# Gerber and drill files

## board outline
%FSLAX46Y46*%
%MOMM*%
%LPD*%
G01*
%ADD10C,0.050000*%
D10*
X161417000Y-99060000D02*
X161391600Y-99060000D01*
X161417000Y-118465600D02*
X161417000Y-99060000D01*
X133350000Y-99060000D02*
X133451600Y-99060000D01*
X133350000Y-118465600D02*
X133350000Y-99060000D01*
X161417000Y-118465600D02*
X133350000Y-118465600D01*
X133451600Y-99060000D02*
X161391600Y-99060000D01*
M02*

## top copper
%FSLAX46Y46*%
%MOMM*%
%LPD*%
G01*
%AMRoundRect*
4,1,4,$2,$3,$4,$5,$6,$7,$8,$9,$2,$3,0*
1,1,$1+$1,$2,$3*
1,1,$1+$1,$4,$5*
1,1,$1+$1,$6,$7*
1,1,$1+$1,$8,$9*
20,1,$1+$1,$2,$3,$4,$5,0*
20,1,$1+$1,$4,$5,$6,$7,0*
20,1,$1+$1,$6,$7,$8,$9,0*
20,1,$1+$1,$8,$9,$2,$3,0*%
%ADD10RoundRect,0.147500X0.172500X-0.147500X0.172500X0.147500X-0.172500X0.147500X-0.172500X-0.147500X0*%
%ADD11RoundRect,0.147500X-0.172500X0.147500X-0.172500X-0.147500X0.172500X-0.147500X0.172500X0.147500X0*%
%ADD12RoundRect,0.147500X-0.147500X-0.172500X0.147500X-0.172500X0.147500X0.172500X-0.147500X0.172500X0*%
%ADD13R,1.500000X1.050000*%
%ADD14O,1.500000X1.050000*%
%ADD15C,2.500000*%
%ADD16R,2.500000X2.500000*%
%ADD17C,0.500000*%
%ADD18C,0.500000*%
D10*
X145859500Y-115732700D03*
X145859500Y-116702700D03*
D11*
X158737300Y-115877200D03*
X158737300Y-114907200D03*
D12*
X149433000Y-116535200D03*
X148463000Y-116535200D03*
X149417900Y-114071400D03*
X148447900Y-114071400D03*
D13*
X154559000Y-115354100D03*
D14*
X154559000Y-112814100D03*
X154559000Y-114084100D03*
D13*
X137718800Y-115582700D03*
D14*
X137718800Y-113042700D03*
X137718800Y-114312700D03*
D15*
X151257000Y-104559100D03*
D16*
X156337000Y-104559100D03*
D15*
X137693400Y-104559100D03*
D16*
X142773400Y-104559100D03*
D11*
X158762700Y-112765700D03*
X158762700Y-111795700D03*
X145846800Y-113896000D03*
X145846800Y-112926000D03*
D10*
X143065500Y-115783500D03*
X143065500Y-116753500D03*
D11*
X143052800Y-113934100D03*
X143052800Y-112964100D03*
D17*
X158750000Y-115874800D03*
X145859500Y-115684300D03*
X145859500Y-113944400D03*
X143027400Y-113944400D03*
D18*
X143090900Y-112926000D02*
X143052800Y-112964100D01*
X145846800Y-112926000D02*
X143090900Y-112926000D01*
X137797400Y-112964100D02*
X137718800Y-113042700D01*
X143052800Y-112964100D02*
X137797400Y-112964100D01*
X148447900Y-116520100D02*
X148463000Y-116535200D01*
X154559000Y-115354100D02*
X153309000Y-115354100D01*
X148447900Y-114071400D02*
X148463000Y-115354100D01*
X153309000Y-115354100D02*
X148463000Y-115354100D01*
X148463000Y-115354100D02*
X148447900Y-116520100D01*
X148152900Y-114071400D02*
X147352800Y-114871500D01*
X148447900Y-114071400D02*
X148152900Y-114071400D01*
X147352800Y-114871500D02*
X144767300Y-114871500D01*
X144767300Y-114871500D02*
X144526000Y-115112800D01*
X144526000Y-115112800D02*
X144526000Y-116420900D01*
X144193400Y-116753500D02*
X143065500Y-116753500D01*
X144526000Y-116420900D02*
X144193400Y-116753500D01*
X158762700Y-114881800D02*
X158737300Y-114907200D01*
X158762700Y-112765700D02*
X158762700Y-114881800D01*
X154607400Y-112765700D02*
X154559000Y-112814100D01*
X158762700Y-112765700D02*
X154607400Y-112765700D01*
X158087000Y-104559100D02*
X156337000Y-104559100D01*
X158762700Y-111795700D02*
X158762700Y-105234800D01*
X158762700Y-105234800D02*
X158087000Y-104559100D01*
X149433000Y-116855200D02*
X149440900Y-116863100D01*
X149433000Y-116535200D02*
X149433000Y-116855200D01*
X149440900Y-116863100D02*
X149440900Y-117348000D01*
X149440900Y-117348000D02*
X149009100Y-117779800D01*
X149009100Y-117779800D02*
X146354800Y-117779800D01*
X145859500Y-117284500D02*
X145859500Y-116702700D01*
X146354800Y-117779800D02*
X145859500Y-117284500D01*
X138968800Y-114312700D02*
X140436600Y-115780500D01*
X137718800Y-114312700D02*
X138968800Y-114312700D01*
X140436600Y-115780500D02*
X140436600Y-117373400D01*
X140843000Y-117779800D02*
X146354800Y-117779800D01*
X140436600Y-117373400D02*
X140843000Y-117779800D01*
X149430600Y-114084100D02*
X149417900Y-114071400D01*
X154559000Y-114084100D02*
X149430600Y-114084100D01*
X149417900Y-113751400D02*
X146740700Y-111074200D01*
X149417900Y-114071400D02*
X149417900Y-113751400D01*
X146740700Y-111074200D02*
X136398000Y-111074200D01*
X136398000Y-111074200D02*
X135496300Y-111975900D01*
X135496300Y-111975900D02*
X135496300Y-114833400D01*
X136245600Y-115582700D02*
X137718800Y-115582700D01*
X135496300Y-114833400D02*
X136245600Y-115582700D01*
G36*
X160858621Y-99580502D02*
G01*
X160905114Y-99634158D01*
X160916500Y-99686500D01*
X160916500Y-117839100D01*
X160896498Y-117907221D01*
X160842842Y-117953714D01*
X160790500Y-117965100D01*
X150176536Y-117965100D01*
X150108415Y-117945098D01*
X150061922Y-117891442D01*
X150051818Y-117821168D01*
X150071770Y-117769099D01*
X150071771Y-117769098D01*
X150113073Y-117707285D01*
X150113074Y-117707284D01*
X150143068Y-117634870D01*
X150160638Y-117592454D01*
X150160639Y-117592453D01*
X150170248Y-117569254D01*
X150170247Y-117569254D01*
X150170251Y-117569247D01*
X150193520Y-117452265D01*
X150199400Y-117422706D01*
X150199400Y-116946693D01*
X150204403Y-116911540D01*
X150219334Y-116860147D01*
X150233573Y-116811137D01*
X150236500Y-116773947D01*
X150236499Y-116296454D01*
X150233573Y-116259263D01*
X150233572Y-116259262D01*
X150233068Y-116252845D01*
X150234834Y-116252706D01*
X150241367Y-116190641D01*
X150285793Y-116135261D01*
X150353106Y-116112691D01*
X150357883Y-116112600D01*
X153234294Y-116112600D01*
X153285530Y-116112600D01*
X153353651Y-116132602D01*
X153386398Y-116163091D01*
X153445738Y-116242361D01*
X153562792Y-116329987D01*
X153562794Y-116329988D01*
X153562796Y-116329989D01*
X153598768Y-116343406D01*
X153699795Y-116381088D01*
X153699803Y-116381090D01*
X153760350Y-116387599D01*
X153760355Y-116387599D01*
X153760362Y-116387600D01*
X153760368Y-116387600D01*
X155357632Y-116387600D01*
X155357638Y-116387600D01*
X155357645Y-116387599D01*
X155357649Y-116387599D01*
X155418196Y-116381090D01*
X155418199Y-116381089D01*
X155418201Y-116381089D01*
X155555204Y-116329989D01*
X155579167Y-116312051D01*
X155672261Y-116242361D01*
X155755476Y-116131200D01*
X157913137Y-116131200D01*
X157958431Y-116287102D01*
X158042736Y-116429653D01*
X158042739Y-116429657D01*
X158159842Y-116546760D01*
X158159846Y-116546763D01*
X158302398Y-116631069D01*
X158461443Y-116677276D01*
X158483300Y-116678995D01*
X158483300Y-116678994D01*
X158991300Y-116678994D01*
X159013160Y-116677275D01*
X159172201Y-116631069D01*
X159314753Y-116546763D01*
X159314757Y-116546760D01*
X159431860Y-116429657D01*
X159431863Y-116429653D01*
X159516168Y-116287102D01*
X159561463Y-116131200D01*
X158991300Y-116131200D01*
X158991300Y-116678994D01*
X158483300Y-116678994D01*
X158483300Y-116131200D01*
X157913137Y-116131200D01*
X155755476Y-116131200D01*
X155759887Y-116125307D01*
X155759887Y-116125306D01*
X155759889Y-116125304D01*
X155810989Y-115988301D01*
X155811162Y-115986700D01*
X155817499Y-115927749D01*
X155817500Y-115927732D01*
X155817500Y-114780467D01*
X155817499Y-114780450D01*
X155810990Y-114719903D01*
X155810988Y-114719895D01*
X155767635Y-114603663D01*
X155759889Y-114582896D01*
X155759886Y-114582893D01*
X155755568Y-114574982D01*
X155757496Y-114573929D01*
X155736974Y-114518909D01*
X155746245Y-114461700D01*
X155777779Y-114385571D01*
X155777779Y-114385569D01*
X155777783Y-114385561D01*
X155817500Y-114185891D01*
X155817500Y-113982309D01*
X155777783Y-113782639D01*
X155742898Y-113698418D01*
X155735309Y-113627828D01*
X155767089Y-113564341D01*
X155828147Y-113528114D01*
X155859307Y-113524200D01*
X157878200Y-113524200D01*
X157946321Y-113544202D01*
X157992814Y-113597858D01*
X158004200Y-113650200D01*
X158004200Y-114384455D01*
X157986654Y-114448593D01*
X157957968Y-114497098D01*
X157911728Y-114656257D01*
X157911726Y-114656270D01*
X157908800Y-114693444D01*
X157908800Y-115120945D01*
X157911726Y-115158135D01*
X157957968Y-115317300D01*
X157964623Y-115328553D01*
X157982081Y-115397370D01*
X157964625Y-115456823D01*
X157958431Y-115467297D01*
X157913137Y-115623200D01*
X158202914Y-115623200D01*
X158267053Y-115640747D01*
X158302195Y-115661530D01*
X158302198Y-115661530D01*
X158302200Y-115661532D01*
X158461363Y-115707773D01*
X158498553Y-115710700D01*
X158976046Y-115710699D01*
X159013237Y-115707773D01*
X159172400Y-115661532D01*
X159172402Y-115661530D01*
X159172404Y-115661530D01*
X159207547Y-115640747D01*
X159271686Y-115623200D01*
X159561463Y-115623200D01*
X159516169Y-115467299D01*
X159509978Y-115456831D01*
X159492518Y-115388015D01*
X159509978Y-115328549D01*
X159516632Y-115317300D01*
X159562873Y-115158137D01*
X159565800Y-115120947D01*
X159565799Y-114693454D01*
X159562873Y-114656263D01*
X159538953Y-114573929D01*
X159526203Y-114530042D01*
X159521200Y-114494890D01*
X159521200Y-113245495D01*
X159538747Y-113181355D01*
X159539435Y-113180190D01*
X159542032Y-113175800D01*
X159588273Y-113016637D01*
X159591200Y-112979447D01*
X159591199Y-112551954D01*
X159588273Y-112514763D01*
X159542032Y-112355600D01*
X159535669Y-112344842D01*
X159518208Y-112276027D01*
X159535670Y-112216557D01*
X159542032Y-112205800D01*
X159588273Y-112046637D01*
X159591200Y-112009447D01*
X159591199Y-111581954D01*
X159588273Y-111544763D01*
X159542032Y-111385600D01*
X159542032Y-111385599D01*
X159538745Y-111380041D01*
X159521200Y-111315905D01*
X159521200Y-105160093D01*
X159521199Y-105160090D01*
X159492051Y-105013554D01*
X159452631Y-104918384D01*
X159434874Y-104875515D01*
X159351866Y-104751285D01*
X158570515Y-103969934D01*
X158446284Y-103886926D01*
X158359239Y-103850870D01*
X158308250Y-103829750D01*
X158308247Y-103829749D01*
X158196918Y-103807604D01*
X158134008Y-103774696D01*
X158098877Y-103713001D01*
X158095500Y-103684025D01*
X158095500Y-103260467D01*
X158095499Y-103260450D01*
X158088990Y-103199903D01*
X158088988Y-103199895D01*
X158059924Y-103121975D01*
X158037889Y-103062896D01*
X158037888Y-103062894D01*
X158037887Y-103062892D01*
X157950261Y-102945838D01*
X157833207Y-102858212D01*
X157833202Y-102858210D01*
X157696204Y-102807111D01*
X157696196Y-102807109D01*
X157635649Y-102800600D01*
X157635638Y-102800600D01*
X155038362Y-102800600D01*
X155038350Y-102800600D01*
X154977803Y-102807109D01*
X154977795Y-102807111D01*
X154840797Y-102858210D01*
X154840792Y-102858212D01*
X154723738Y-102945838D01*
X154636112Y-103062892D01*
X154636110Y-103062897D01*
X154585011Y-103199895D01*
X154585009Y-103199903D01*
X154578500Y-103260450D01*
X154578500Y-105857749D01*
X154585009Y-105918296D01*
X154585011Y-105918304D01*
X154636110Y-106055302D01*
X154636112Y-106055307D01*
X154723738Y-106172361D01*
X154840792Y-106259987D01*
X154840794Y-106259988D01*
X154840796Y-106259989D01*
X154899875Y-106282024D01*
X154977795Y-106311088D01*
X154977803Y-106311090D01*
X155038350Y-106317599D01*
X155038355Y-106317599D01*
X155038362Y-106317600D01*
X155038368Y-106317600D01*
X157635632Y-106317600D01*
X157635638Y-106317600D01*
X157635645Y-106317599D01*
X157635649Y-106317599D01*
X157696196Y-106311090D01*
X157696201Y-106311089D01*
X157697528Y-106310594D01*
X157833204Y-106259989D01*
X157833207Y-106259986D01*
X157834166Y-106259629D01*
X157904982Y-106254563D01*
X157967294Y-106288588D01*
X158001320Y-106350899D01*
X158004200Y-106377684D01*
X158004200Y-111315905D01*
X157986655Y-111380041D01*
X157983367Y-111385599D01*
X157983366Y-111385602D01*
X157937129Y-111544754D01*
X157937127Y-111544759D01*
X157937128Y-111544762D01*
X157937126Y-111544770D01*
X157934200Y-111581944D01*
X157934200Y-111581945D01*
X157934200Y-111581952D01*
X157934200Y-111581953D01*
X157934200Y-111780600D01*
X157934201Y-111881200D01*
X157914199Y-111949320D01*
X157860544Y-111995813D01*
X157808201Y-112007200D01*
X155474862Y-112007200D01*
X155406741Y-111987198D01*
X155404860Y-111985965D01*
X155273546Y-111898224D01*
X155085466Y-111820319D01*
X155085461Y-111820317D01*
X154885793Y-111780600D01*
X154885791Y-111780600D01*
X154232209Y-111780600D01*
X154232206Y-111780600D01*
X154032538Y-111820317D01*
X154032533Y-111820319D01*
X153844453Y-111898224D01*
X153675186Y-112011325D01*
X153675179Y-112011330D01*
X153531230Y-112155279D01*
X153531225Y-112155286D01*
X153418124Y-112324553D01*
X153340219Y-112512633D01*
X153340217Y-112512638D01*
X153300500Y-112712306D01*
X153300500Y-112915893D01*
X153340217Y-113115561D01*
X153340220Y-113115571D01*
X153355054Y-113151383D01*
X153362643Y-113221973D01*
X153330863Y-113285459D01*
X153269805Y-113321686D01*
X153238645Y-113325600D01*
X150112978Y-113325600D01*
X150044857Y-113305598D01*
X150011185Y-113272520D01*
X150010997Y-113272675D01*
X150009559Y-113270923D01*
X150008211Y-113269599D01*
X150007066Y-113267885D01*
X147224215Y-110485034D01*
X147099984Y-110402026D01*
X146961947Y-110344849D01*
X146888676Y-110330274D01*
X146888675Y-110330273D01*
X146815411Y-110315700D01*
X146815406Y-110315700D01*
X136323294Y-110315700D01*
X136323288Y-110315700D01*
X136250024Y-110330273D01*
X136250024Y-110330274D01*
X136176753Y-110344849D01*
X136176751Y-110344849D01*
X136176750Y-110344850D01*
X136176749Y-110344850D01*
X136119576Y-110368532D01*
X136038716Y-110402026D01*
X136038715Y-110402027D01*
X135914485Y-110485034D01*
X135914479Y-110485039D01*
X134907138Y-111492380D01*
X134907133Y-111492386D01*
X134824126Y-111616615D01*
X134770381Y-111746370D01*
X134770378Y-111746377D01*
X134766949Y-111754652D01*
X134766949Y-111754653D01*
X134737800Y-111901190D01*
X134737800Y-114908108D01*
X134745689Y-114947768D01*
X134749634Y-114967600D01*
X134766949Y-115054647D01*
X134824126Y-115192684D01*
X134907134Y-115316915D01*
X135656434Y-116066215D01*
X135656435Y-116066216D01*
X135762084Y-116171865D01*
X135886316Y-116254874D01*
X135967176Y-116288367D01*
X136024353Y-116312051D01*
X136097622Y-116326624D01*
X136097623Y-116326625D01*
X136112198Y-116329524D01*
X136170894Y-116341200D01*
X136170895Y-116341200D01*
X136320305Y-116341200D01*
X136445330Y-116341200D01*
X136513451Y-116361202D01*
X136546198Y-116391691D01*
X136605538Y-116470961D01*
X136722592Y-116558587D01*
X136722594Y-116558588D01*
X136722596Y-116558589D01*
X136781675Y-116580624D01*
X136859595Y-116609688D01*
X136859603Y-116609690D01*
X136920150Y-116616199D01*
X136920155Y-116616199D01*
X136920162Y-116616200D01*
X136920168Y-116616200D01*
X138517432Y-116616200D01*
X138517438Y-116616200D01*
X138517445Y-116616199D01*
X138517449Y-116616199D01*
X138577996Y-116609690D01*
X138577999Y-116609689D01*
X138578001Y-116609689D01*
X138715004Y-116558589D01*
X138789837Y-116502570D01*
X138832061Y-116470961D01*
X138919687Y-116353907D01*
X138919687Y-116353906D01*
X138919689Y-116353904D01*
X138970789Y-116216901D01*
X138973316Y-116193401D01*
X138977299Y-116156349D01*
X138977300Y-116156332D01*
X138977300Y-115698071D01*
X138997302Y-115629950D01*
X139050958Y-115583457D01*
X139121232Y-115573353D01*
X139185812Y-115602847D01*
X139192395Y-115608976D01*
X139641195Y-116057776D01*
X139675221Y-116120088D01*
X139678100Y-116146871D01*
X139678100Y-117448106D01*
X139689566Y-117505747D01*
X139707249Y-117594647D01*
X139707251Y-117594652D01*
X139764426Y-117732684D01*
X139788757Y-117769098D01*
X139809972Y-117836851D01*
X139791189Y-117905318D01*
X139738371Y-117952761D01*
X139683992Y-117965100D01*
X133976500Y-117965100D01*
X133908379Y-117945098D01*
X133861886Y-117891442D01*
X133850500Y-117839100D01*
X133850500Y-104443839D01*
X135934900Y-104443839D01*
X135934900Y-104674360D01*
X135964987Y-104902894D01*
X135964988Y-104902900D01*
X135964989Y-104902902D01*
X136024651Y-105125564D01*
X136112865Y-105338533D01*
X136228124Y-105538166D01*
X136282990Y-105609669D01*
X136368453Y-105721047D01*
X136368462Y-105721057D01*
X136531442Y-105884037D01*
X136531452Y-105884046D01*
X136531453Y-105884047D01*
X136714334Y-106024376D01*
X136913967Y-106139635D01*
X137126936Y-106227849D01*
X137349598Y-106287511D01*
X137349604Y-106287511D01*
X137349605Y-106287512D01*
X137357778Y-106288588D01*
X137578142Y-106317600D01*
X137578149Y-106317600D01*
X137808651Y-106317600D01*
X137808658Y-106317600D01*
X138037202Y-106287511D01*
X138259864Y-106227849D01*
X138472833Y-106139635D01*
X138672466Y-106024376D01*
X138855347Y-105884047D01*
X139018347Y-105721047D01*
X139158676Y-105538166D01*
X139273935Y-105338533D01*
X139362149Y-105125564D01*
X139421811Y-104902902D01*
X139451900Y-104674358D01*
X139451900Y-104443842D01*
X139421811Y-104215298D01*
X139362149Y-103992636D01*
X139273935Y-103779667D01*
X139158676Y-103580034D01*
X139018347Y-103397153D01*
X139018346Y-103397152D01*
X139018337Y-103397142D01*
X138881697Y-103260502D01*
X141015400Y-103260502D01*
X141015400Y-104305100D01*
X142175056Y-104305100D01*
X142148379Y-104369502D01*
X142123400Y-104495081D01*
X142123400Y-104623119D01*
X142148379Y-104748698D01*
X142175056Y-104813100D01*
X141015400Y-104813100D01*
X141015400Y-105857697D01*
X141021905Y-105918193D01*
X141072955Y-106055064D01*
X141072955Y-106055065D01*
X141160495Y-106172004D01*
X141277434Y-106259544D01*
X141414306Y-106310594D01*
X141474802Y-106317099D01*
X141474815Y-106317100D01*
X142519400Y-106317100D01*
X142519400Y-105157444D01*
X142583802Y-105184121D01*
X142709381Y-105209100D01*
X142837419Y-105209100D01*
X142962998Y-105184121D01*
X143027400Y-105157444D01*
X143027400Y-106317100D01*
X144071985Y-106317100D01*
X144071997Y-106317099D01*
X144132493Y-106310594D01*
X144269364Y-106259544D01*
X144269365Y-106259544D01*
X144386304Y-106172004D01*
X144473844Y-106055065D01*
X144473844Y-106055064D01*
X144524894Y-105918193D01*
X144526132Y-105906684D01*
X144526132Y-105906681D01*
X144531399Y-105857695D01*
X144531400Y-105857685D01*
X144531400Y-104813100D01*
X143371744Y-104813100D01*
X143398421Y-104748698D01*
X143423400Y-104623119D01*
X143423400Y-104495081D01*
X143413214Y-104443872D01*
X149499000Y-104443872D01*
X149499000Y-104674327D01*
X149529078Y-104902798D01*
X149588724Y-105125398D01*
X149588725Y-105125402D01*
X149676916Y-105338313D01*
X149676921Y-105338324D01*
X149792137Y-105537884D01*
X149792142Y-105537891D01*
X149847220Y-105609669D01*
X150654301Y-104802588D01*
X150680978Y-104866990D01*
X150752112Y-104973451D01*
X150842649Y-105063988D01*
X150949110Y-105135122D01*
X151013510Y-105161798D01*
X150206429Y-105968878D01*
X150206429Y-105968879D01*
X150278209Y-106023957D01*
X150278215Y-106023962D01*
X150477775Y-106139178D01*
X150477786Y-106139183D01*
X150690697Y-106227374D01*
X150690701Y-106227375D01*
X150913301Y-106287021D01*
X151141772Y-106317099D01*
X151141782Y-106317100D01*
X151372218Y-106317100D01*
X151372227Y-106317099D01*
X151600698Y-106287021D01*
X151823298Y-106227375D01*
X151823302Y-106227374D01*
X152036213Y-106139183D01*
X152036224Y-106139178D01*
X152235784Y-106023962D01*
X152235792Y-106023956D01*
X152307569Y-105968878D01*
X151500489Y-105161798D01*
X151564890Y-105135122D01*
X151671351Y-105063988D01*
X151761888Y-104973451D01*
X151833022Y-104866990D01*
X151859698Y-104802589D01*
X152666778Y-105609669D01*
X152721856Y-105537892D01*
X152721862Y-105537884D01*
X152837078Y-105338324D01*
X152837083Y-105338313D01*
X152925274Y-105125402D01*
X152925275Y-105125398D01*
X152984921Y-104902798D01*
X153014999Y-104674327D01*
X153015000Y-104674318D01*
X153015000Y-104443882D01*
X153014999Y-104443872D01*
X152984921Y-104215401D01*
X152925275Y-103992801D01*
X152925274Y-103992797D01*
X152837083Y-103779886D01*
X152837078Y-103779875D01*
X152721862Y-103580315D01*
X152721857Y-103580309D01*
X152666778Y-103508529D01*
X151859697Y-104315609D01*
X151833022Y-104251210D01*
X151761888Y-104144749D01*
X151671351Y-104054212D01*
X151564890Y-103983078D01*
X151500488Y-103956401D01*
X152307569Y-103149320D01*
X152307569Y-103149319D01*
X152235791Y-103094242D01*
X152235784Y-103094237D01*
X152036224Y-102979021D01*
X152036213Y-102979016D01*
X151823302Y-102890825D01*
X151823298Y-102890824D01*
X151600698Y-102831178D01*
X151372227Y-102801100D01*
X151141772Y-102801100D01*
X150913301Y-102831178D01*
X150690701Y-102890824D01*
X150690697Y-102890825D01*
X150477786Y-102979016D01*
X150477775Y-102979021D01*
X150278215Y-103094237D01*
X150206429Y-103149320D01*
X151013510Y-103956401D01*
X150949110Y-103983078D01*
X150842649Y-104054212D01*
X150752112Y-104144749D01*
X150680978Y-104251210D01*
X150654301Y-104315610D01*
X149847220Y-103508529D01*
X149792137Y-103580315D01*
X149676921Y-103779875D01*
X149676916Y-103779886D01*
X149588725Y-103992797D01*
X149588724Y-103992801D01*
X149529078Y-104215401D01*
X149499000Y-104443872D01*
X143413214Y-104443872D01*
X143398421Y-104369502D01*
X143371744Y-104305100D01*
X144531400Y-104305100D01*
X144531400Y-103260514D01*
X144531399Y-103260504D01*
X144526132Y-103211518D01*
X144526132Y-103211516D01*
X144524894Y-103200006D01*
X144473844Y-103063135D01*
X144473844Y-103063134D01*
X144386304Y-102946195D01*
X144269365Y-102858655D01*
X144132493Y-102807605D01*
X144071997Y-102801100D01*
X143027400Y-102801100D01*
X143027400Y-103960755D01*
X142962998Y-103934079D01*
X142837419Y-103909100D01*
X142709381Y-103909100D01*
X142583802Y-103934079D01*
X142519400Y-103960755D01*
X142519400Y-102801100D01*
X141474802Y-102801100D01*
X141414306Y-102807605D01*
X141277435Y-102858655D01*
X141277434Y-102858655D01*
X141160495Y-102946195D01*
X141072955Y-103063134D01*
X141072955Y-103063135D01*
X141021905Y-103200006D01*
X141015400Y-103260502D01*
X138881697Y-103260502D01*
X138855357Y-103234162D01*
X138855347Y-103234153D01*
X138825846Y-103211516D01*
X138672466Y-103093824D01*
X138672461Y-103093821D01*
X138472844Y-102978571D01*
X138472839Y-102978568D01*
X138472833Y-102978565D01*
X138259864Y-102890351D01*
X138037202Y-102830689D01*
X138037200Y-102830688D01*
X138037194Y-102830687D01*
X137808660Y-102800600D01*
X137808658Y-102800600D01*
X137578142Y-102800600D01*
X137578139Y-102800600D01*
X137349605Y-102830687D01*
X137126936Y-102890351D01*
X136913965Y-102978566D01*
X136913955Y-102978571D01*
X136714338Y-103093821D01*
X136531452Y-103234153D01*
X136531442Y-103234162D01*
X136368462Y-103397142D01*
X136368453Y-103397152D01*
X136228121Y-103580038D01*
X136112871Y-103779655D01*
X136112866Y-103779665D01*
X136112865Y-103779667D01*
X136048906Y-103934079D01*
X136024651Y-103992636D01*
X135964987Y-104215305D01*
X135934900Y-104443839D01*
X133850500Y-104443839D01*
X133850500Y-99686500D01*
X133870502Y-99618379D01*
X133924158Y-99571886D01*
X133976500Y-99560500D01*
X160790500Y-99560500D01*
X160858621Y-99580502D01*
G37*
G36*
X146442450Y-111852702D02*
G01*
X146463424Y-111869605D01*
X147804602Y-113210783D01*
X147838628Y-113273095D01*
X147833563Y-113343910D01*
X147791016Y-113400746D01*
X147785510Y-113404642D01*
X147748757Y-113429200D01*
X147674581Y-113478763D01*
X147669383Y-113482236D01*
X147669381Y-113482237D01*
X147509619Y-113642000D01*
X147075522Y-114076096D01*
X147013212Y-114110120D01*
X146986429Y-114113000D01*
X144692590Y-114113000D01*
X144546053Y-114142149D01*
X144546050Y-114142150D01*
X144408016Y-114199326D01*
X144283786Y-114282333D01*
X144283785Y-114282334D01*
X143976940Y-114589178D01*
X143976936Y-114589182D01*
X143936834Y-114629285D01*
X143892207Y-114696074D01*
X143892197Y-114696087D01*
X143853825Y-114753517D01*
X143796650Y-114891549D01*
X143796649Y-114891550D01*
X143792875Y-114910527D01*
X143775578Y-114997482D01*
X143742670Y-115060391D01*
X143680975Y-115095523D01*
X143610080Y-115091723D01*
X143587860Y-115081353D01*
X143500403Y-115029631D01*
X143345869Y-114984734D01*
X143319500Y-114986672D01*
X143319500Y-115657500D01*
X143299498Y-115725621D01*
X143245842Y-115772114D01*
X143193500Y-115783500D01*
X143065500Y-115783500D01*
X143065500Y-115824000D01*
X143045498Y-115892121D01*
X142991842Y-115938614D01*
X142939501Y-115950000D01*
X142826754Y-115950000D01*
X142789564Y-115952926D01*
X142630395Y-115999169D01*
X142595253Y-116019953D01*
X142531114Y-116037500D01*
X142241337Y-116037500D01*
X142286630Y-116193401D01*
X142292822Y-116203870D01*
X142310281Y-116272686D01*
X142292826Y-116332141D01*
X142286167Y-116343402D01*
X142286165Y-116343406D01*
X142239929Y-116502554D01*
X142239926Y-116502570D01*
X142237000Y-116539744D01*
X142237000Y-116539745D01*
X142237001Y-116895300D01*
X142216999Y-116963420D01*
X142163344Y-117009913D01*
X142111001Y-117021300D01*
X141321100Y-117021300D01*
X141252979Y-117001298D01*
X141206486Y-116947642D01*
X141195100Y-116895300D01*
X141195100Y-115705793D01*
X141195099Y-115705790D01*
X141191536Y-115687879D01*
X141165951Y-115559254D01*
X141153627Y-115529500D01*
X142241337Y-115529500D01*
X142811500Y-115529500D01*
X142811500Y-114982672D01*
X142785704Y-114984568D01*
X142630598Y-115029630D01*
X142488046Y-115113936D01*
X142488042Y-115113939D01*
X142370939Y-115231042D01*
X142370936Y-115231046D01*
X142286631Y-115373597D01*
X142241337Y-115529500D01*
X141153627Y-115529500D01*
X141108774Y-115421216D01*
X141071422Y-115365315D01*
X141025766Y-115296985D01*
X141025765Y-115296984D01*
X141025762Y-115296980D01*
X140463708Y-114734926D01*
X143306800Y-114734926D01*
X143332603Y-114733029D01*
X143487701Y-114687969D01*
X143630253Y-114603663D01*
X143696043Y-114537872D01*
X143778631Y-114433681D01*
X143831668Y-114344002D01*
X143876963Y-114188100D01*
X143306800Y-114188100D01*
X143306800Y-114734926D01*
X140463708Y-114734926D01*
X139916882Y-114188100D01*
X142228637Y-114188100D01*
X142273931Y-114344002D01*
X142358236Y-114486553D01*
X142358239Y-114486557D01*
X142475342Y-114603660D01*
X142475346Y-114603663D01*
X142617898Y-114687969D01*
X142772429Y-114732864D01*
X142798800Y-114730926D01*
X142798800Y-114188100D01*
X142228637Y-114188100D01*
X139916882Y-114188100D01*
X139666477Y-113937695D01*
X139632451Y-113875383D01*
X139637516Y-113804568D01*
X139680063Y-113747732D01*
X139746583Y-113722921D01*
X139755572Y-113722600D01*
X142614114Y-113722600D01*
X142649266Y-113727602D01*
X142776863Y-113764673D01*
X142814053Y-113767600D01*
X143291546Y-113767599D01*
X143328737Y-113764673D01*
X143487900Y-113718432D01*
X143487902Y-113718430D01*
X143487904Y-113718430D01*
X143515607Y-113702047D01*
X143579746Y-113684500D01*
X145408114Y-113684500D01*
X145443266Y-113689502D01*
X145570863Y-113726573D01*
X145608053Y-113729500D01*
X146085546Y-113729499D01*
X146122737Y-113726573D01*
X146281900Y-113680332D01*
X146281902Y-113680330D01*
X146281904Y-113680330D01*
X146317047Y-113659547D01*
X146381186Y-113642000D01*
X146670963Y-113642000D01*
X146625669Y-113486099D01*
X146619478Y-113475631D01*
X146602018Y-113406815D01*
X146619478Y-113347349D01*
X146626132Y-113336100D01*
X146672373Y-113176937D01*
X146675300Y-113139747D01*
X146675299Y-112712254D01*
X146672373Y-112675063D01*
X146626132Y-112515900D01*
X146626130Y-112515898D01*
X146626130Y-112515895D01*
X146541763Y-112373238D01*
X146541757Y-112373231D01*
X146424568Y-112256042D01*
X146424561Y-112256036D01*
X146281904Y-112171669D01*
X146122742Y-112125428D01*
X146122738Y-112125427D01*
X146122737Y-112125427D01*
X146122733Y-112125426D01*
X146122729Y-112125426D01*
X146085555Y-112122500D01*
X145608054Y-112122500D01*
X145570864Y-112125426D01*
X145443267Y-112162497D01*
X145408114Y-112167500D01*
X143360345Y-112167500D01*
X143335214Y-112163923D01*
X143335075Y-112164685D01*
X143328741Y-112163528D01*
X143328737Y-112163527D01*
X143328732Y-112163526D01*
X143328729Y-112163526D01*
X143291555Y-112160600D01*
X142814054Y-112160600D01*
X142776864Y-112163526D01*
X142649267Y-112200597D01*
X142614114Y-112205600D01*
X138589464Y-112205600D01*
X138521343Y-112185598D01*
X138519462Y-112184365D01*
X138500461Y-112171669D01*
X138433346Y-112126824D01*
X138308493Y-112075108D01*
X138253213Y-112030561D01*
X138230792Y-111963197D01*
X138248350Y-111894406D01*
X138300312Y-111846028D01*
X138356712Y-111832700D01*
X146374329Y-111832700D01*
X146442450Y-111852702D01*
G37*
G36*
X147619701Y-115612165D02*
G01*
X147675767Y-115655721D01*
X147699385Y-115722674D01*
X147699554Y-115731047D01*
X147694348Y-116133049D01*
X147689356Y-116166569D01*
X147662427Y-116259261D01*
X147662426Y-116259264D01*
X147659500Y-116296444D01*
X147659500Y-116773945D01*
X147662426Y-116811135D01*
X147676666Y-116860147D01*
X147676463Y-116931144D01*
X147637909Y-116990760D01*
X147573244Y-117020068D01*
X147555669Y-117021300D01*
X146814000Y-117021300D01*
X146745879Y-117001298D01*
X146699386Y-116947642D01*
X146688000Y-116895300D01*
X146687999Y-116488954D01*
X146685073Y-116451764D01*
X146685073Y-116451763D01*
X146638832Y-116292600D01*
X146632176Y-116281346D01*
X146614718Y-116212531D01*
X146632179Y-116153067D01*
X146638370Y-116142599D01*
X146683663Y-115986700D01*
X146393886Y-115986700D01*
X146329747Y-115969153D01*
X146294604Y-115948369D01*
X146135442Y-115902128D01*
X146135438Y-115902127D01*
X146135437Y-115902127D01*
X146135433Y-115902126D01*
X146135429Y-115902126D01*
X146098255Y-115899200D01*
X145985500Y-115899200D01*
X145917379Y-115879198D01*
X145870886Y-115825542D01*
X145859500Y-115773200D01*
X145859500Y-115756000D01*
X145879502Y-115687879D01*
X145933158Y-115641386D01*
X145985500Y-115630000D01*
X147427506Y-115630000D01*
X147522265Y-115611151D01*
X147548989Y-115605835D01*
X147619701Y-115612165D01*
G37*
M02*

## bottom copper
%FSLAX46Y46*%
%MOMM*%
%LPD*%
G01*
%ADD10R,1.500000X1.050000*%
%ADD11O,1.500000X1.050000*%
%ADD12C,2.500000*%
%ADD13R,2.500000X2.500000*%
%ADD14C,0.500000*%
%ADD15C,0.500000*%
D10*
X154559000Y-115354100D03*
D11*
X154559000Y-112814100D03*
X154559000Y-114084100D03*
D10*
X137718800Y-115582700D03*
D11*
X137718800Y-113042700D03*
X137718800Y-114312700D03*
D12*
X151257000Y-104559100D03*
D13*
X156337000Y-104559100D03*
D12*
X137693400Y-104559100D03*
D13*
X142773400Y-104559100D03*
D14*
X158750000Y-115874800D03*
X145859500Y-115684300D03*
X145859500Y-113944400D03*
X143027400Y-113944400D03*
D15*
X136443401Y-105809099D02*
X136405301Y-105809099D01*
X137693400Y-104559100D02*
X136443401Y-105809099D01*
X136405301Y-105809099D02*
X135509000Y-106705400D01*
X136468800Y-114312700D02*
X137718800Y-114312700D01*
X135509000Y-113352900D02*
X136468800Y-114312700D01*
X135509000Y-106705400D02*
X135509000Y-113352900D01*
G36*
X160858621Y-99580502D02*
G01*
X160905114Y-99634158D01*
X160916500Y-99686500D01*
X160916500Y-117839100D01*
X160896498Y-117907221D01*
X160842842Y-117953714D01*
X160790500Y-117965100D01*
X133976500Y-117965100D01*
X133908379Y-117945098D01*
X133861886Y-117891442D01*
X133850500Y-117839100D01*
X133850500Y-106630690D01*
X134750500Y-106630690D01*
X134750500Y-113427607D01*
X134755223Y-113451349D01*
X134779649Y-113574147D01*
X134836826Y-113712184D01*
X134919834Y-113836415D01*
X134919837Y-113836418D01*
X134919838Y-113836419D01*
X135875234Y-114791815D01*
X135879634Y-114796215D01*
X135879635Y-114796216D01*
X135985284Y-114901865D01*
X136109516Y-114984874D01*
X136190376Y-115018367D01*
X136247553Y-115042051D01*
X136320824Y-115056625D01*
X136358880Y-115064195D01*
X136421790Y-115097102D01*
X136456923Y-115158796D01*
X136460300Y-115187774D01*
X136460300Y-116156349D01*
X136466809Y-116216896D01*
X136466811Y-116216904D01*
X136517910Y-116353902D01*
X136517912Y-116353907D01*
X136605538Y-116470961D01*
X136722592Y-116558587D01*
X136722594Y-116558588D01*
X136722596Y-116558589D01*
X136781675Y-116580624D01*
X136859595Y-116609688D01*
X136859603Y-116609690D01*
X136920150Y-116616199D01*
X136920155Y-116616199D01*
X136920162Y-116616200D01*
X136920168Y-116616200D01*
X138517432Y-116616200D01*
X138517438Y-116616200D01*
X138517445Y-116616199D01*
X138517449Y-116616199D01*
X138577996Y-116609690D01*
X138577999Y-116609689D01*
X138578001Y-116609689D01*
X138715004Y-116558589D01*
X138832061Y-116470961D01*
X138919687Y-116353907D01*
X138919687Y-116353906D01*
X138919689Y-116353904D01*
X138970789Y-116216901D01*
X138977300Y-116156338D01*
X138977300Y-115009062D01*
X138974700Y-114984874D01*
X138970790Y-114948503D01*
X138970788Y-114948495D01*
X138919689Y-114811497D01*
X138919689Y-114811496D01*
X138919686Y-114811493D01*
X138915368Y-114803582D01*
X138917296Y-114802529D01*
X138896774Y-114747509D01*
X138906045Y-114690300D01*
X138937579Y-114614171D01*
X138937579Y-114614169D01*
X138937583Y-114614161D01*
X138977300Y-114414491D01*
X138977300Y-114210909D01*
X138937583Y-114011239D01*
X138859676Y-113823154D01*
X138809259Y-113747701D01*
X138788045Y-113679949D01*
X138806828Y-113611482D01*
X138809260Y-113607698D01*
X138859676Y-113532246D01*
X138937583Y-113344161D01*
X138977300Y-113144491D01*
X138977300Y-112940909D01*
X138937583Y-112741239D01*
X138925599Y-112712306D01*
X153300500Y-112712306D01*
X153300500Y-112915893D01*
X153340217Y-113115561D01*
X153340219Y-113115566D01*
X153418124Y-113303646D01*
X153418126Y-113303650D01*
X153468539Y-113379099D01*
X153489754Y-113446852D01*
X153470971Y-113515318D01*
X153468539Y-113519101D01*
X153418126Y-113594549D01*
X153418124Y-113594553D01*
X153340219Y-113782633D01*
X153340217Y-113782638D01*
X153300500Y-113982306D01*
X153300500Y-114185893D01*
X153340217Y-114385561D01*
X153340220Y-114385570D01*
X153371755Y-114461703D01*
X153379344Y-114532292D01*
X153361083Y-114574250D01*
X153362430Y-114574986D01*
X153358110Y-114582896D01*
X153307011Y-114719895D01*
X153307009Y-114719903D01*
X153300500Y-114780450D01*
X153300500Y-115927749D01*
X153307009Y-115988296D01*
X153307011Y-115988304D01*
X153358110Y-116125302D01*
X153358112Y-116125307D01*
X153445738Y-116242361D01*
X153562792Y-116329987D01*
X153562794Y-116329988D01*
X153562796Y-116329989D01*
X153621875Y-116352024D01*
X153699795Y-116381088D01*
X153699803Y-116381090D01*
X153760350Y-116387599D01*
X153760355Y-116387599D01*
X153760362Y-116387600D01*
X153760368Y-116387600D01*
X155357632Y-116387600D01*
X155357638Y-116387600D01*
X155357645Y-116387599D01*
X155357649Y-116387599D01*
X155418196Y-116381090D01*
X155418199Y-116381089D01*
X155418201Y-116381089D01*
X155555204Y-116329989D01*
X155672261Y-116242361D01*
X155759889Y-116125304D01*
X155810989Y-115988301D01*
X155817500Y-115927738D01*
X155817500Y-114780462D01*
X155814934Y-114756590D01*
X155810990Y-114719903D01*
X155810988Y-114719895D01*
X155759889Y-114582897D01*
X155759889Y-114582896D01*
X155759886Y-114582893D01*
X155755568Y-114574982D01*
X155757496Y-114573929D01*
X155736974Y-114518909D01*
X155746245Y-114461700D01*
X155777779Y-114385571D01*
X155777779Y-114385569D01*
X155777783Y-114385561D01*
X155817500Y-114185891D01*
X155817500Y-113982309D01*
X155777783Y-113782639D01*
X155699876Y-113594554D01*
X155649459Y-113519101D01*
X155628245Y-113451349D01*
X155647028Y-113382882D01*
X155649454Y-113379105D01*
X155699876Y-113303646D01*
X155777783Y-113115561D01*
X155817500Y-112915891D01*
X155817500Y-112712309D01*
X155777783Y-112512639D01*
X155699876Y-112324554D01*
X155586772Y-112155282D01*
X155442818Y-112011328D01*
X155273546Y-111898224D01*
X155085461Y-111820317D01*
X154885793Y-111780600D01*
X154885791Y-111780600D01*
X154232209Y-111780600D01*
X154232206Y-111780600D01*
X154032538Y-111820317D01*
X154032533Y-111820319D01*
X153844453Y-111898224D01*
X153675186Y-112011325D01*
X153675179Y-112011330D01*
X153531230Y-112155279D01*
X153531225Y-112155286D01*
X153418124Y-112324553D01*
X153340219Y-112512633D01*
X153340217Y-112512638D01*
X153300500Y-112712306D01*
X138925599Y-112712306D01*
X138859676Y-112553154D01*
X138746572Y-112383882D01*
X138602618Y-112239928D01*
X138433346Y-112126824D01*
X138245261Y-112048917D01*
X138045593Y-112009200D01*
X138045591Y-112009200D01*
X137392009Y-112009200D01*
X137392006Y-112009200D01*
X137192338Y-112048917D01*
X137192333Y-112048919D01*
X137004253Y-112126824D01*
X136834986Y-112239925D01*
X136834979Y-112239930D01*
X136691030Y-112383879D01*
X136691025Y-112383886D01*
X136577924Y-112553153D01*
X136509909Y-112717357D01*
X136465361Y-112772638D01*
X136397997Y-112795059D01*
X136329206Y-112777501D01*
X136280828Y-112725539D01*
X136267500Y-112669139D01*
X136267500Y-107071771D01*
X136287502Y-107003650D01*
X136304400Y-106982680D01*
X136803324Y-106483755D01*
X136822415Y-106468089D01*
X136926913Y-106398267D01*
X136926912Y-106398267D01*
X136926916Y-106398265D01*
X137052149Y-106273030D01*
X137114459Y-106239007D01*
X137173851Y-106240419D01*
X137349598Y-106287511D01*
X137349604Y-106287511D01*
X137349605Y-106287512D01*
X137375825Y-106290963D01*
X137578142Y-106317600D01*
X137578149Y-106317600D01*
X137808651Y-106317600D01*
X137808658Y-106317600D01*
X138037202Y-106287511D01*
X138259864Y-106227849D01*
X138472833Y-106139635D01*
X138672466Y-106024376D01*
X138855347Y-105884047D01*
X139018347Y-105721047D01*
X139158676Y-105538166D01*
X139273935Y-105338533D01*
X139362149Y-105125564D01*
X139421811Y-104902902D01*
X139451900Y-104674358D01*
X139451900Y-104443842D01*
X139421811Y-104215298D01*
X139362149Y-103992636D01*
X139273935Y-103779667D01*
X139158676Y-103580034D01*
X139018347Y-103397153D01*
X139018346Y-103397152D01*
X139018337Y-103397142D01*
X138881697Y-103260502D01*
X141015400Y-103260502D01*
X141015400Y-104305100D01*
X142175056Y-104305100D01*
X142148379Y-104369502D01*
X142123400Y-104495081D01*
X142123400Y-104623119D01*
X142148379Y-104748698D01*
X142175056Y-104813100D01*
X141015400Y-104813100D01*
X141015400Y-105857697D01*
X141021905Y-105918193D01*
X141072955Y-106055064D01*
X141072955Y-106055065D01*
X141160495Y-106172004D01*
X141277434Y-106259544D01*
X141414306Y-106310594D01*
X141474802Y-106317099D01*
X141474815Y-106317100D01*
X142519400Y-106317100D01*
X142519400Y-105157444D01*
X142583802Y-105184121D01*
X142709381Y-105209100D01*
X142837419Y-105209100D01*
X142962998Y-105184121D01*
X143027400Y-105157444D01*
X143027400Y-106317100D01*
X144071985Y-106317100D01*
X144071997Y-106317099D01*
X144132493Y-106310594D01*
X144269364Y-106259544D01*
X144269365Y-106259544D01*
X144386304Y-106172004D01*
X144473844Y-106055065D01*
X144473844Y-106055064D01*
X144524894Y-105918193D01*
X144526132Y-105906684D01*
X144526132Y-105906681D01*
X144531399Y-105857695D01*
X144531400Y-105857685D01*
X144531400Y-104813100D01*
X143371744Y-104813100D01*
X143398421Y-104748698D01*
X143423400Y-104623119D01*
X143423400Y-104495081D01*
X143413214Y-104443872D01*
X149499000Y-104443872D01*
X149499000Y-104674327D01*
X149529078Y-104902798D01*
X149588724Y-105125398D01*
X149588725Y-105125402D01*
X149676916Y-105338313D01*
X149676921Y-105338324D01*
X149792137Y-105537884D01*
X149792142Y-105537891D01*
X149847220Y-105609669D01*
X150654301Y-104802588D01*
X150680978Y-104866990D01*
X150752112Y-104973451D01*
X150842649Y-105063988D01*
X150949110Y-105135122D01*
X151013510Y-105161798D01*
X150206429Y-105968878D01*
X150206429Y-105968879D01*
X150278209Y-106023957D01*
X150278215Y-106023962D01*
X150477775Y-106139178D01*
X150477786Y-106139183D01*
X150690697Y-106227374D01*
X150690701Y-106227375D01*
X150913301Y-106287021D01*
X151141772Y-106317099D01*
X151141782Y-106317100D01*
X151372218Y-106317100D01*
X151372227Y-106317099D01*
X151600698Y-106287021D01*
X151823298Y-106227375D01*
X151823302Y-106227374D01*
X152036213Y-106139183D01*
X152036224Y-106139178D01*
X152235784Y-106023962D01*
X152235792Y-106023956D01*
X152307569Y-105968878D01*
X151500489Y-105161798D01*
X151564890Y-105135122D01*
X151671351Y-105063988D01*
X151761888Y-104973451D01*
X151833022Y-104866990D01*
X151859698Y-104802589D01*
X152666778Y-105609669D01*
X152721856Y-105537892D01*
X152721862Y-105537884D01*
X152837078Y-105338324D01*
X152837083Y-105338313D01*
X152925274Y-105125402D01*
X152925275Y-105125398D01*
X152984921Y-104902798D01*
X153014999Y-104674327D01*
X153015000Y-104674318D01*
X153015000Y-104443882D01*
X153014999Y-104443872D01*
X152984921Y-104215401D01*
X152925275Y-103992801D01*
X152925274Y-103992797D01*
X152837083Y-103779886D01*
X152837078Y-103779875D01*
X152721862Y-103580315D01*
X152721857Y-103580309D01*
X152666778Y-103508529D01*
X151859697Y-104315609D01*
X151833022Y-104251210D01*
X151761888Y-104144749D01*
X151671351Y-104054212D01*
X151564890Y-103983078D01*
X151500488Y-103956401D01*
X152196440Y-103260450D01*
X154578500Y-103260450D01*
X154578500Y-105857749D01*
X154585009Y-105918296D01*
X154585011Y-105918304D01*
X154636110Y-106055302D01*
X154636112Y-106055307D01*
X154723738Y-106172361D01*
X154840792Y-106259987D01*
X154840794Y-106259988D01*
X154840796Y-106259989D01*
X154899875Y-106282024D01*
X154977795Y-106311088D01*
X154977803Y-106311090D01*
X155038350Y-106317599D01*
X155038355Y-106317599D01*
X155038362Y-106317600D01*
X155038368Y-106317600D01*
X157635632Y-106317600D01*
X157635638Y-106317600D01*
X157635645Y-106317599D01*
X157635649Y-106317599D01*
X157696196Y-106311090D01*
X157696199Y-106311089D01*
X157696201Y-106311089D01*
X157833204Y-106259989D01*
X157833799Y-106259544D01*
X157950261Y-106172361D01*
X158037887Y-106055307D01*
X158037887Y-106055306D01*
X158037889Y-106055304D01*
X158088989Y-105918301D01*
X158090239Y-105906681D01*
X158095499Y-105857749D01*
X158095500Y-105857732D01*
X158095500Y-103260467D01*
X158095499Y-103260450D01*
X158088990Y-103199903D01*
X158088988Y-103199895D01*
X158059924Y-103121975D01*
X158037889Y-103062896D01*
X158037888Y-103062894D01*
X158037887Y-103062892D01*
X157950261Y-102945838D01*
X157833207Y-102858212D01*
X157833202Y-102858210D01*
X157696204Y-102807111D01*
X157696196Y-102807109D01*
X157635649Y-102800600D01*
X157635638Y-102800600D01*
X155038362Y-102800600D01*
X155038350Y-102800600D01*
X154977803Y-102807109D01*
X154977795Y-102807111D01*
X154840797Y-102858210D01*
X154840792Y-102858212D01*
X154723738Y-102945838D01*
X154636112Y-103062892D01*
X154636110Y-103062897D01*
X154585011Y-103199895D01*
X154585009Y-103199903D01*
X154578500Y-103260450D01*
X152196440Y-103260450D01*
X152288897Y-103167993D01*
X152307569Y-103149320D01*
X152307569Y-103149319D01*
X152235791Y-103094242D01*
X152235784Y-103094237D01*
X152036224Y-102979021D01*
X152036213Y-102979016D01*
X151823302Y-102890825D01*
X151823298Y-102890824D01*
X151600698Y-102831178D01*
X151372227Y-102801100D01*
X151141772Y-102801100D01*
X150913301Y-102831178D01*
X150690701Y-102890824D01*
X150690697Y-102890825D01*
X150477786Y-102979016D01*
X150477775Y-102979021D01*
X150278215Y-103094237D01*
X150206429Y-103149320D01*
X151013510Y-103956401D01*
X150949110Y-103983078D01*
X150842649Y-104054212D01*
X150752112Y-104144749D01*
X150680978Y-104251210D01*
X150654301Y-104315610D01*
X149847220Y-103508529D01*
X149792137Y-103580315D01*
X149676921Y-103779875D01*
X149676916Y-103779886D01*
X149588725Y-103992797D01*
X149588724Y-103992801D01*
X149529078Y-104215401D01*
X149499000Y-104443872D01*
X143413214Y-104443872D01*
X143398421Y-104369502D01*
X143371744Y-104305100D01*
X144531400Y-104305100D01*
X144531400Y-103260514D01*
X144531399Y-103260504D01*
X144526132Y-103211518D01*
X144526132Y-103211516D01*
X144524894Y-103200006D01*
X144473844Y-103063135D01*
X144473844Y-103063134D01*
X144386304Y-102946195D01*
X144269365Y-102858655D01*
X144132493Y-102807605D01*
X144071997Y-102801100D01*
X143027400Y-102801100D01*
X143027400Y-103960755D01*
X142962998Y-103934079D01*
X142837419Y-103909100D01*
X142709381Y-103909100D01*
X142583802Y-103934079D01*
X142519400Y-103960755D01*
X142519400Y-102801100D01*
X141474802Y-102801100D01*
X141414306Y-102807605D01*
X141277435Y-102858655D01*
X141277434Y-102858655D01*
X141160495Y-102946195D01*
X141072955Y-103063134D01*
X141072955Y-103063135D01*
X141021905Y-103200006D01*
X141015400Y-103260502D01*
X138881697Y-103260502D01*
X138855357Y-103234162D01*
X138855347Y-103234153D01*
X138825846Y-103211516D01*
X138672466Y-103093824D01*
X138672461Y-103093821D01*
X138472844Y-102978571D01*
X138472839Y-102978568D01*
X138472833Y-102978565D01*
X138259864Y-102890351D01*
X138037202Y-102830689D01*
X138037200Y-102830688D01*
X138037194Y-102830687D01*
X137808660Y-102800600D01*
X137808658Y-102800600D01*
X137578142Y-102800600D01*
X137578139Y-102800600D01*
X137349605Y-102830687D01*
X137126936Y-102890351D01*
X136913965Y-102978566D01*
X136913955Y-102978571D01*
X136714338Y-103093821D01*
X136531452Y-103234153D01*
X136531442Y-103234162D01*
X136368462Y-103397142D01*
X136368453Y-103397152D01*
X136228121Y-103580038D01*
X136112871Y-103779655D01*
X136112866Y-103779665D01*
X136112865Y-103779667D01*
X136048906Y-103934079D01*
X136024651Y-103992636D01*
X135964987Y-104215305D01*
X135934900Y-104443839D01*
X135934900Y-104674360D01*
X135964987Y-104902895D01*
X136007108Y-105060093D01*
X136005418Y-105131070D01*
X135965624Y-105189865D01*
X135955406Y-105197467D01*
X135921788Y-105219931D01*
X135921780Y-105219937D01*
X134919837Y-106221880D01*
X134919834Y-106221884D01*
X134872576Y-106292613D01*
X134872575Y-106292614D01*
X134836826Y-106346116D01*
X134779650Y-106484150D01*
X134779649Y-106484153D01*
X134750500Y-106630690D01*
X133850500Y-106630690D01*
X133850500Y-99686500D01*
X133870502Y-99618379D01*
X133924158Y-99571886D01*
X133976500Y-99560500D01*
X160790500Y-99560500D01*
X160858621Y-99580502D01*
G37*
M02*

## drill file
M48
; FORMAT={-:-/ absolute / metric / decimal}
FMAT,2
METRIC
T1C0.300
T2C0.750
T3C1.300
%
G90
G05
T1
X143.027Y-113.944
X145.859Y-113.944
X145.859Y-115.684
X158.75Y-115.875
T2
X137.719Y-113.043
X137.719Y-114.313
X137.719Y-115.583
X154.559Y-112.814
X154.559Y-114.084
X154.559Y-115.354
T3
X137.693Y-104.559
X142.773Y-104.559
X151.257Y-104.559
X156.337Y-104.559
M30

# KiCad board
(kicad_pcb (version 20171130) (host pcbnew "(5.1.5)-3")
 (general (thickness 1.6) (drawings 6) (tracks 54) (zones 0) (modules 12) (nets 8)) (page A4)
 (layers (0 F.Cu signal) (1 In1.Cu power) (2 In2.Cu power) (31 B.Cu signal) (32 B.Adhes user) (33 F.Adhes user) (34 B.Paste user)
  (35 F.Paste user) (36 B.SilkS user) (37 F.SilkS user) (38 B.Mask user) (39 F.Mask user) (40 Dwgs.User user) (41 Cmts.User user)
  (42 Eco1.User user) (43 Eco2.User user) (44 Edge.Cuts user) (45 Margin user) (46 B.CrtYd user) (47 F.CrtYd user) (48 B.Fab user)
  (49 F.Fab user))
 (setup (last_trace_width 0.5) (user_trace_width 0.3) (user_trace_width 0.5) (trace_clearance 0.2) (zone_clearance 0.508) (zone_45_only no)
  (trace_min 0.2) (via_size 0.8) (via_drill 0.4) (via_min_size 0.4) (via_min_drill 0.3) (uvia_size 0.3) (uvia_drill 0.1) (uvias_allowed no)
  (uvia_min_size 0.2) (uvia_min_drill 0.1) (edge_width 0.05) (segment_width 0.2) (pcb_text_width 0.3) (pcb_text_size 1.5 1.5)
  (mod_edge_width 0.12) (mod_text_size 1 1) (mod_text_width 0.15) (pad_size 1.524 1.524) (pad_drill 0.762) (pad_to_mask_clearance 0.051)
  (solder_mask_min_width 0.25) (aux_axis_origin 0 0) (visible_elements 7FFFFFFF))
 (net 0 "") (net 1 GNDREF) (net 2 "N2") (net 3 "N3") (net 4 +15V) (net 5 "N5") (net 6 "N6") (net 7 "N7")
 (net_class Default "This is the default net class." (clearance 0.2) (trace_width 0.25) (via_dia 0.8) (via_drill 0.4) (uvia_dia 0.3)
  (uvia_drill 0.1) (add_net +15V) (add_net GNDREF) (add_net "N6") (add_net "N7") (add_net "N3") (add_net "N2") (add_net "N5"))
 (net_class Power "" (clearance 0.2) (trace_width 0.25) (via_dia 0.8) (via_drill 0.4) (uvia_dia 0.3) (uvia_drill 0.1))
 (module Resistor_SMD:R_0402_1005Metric (layer F.Cu) (at 145.8595 116.2177 90)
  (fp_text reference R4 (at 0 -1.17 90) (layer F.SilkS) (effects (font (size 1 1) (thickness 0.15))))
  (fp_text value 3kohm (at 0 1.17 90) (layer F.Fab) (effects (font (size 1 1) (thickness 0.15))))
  (pad 2 smd roundrect (at 0.485 0 90) (size 0.59 0.64) (layers F.Cu F.Paste F.Mask) (roundrect_rratio 0.25) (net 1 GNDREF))
  (pad 1 smd roundrect (at -0.485 0 90) (size 0.59 0.64) (layers F.Cu F.Paste F.Mask) (roundrect_rratio 0.25) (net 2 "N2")))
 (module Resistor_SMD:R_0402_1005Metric (layer F.Cu) (at 158.7373 115.3922 270)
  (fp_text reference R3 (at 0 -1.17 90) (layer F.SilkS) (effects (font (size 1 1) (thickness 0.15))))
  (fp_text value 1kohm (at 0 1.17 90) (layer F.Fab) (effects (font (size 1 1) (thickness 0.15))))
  (pad 2 smd roundrect (at 0.485 0 270) (size 0.59 0.64) (layers F.Cu F.Paste F.Mask) (roundrect_rratio 0.25) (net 1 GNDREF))
  (pad 1 smd roundrect (at -0.485 0 270) (size 0.59 0.64) (layers F.Cu F.Paste F.Mask) (roundrect_rratio 0.25) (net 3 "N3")))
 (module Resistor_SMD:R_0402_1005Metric (layer F.Cu) (at 148.948 116.5352)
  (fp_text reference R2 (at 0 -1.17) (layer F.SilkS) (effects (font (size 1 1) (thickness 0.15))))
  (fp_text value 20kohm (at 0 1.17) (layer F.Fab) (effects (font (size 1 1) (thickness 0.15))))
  (pad 2 smd roundrect (at 0.485 0) (size 0.59 0.64) (layers F.Cu F.Paste F.Mask) (roundrect_rratio 0.25) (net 2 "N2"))
  (pad 1 smd roundrect (at -0.485 0) (size 0.59 0.64) (layers F.Cu F.Paste F.Mask) (roundrect_rratio 0.25) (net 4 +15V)))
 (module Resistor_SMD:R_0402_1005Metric (layer F.Cu) (at 148.9329 114.0714)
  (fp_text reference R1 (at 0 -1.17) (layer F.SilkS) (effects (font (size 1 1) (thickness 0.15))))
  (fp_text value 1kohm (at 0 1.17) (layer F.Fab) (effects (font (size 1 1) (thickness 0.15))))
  (pad 2 smd roundrect (at 0.485 0) (size 0.59 0.64) (layers F.Cu F.Paste F.Mask) (roundrect_rratio 0.25) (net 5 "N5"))
  (pad 1 smd roundrect (at -0.485 0) (size 0.59 0.64) (layers F.Cu F.Paste F.Mask) (roundrect_rratio 0.25) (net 4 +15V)))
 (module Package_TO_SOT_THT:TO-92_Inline (layer F.Cu) (at 154.559 115.3541 90)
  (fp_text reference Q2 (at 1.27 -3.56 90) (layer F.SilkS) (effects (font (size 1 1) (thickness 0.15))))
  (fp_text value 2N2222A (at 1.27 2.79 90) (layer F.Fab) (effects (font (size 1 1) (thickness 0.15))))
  (pad 1 thru_hole rect (at 0 0 90) (size 1.05 1.5) (drill 0.75) (layers *.Cu *.Mask) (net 4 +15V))
  (pad 3 thru_hole oval (at 2.54 0 90) (size 1.05 1.5) (drill 0.75) (layers *.Cu *.Mask) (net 3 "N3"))
  (pad 2 thru_hole oval (at 1.27 0 90) (size 1.05 1.5) (drill 0.75) (layers *.Cu *.Mask) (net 5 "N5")))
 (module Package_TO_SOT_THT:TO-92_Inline (layer F.Cu) (at 137.7188 115.5827 90)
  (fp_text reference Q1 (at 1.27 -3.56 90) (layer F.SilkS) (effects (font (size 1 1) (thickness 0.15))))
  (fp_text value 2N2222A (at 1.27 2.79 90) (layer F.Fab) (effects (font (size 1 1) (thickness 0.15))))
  (pad 1 thru_hole rect (at 0 0 90) (size 1.05 1.5) (drill 0.75) (layers *.Cu *.Mask) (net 5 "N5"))
  (pad 3 thru_hole oval (at 2.54 0 90) (size 1.05 1.5) (drill 0.75) (layers *.Cu *.Mask) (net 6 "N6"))
  (pad 2 thru_hole oval (at 1.27 0 90) (size 1.05 1.5) (drill 0.75) (layers *.Cu *.Mask) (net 2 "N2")))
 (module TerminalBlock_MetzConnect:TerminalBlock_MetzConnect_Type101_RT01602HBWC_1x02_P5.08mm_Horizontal (layer F.Cu)
  (at 156.337 104.5591 180)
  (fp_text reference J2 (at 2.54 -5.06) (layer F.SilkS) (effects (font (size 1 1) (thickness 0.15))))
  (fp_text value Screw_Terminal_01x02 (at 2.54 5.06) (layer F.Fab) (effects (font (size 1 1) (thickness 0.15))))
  (pad 2 thru_hole circle (at 5.08 0 180) (size 2.5 2.5) (drill 1.3) (layers *.Cu *.Mask) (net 1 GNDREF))
  (pad 1 thru_hole rect (at 0 0 180) (size 2.5 2.5) (drill 1.3) (layers *.Cu *.Mask) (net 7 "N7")))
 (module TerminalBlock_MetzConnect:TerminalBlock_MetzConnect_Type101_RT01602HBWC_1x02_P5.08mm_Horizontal (layer F.Cu)
  (at 142.7734 104.5591 180)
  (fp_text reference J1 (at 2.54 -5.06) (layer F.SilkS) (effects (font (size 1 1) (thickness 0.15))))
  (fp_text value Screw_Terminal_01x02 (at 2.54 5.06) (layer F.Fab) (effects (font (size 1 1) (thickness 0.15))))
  (pad 2 thru_hole circle (at 5.08 0 180) (size 2.5 2.5) (drill 1.3) (layers *.Cu *.Mask) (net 2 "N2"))
  (pad 1 thru_hole rect (at 0 0 180) (size 2.5 2.5) (drill 1.3) (layers *.Cu *.Mask) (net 1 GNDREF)))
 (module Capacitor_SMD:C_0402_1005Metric (layer F.Cu) (at 158.7627 112.2807 270)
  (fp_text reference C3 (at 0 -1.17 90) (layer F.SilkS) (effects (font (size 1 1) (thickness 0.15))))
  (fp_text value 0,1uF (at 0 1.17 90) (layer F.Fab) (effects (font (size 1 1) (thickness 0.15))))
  (pad 2 smd roundrect (at 0.485 0 270) (size 0.59 0.64) (layers F.Cu F.Paste F.Mask) (roundrect_rratio 0.25) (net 3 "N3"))
  (pad 1 smd roundrect (at -0.485 0 270) (size 0.59 0.64) (layers F.Cu F.Paste F.Mask) (roundrect_rratio 0.25) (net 7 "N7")))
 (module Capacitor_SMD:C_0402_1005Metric (layer F.Cu) (at 145.8468 113.411 270)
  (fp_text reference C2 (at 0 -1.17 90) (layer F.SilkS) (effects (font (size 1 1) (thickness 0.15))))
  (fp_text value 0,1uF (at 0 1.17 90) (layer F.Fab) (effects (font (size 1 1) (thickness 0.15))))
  (pad 2 smd roundrect (at 0.485 0 270) (size 0.59 0.64) (layers F.Cu F.Paste F.Mask) (roundrect_rratio 0.25) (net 1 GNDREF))
  (pad 1 smd roundrect (at -0.485 0 270) (size 0.59 0.64) (layers F.Cu F.Paste F.Mask) (roundrect_rratio 0.25) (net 6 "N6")))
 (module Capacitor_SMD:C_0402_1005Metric (layer F.Cu) (at 143.0655 116.2685 90)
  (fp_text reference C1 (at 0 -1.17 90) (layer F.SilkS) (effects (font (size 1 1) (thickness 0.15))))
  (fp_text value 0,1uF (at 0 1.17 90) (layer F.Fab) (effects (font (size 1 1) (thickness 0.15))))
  (pad 2 smd roundrect (at 0.485 0 90) (size 0.59 0.64) (layers F.Cu F.Paste F.Mask) (roundrect_rratio 0.25) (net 1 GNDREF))
  (pad 1 smd roundrect (at -0.485 0 90) (size 0.59 0.64) (layers F.Cu F.Paste F.Mask) (roundrect_rratio 0.25) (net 4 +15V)))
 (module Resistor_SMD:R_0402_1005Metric (layer F.Cu) (at 143.0528 113.4491 270)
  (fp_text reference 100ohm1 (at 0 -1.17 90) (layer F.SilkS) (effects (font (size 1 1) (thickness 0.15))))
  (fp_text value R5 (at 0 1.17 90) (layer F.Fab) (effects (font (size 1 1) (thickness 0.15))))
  (pad 2 smd roundrect (at 0.485 0 270) (size 0.59 0.64) (layers F.Cu F.Paste F.Mask) (roundrect_rratio 0.25) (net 1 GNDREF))
  (pad 1 smd roundrect (at -0.485 0 270) (size 0.59 0.64) (layers F.Cu F.Paste F.Mask) (roundrect_rratio 0.25) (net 6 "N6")))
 (gr_line (start 161.417 99.06) (end 161.3916 99.06) (layer Edge.Cuts) (width 0.05))
 (gr_line (start 161.417 118.4656) (end 161.417 99.06) (layer Edge.Cuts) (width 0.05))
 (gr_line (start 133.35 99.06) (end 133.4516 99.06) (layer Edge.Cuts) (width 0.05))
 (gr_line (start 133.35 118.4656) (end 133.35 99.06) (layer Edge.Cuts) (width 0.05))
 (gr_line (start 161.417 118.4656) (end 133.35 118.4656) (layer Edge.Cuts) (width 0.05))
 (gr_line (start 133.4516 99.06) (end 161.3916 99.06) (layer Edge.Cuts) (width 0.05))
 (via (at 158.75 115.8748) (size 0.5) (drill 0.3) (layers F.Cu B.Cu) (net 1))
 (via (at 145.8595 115.6843) (size 0.5) (drill 0.3) (layers F.Cu B.Cu) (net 1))
 (via (at 145.8595 113.9444) (size 0.5) (drill 0.3) (layers F.Cu B.Cu) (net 1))
 (via (at 143.0274 113.9444) (size 0.5) (drill 0.3) (layers F.Cu B.Cu) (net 1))
 (segment (start 143.0909 112.926) (end 143.0528 112.9641) (width 0.5) (layer F.Cu) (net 6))
 (segment (start 145.8468 112.926) (end 143.0909 112.926) (width 0.5) (layer F.Cu) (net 6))
 (segment (start 137.7974 112.9641) (end 137.7188 113.0427) (width 0.5) (layer F.Cu) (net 6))
 (segment (start 143.0528 112.9641) (end 137.7974 112.9641) (width 0.5) (layer F.Cu) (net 6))
 (segment (start 148.4479 116.5201) (end 148.463 116.5352) (width 0.5) (layer F.Cu) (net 4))
 (segment (start 154.559 115.3541) (end 153.309 115.3541) (width 0.5) (layer F.Cu) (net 4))
 (segment (start 148.4479 114.0714) (end 148.463 115.3541) (width 0.5) (layer F.Cu) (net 4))
 (segment (start 153.309 115.3541) (end 148.463 115.3541) (width 0.5) (layer F.Cu) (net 4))
 (segment (start 148.463 115.3541) (end 148.4479 116.5201) (width 0.5) (layer F.Cu) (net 4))
 (segment (start 148.1529 114.0714) (end 147.3528 114.8715) (width 0.5) (layer F.Cu) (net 4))
 (segment (start 148.4479 114.0714) (end 148.1529 114.0714) (width 0.5) (layer F.Cu) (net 4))
 (segment (start 147.3528 114.8715) (end 144.7673 114.8715) (width 0.5) (layer F.Cu) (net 4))
 (segment (start 144.7673 114.8715) (end 144.526 115.1128) (width 0.5) (layer F.Cu) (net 4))
 (segment (start 144.526 115.1128) (end 144.526 116.4209) (width 0.5) (layer F.Cu) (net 4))
 (segment (start 144.1934 116.7535) (end 143.0655 116.7535) (width 0.5) (layer F.Cu) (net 4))
 (segment (start 144.526 116.4209) (end 144.1934 116.7535) (width 0.5) (layer F.Cu) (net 4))
 (segment (start 158.7627 114.8818) (end 158.7373 114.9072) (width 0.5) (layer F.Cu) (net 3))
 (segment (start 158.7627 112.7657) (end 158.7627 114.8818) (width 0.5) (layer F.Cu) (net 3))
 (segment (start 154.6074 112.7657) (end 154.559 112.8141) (width 0.5) (layer F.Cu) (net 3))
 (segment (start 158.7627 112.7657) (end 154.6074 112.7657) (width 0.5) (layer F.Cu) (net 3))
 (segment (start 158.087 104.5591) (end 156.337 104.5591) (width 0.5) (layer F.Cu) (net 7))
 (segment (start 158.7627 111.7957) (end 158.7627 105.2348) (width 0.5) (layer F.Cu) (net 7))
 (segment (start 158.7627 105.2348) (end 158.087 104.5591) (width 0.5) (layer F.Cu) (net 7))
 (segment (start 136.443401 105.809099) (end 136.405301 105.809099) (width 0.5) (layer B.Cu) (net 2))
 (segment (start 137.6934 104.5591) (end 136.443401 105.809099) (width 0.5) (layer B.Cu) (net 2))
 (segment (start 136.405301 105.809099) (end 135.509 106.7054) (width 0.5) (layer B.Cu) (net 2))
 (segment (start 136.4688 114.3127) (end 137.7188 114.3127) (width 0.5) (layer B.Cu) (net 2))
 (segment (start 135.509 113.3529) (end 136.4688 114.3127) (width 0.5) (layer B.Cu) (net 2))
 (segment (start 135.509 106.7054) (end 135.509 113.3529) (width 0.5) (layer B.Cu) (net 2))
 (segment (start 149.433 116.8552) (end 149.4409 116.8631) (width 0.5) (layer F.Cu) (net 2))
 (segment (start 149.433 116.5352) (end 149.433 116.8552) (width 0.5) (layer F.Cu) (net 2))
 (segment (start 149.4409 116.8631) (end 149.4409 117.348) (width 0.5) (layer F.Cu) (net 2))
 (segment (start 149.4409 117.348) (end 149.0091 117.7798) (width 0.5) (layer F.Cu) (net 2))
 (segment (start 149.0091 117.7798) (end 146.3548 117.7798) (width 0.5) (layer F.Cu) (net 2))
 (segment (start 145.8595 117.2845) (end 145.8595 116.7027) (width 0.5) (layer F.Cu) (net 2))
 (segment (start 146.3548 117.7798) (end 145.8595 117.2845) (width 0.5) (layer F.Cu) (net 2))
 (segment (start 138.9688 114.3127) (end 140.4366 115.7805) (width 0.5) (layer F.Cu) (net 2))
 (segment (start 137.7188 114.3127) (end 138.9688 114.3127) (width 0.5) (layer F.Cu) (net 2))
 (segment (start 140.4366 115.7805) (end 140.4366 117.3734) (width 0.5) (layer F.Cu) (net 2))
 (segment (start 140.843 117.7798) (end 146.3548 117.7798) (width 0.5) (layer F.Cu) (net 2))
 (segment (start 140.4366 117.3734) (end 140.843 117.7798) (width 0.5) (layer F.Cu) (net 2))
 (segment (start 149.4306 114.0841) (end 149.4179 114.0714) (width 0.5) (layer F.Cu) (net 5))
 (segment (start 154.559 114.0841) (end 149.4306 114.0841) (width 0.5) (layer F.Cu) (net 5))
 (segment (start 149.4179 113.7514) (end 146.7407 111.0742) (width 0.5) (layer F.Cu) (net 5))
 (segment (start 149.4179 114.0714) (end 149.4179 113.7514) (width 0.5) (layer F.Cu) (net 5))
 (segment (start 146.7407 111.0742) (end 136.398 111.0742) (width 0.5) (layer F.Cu) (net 5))
 (segment (start 136.398 111.0742) (end 135.4963 111.9759) (width 0.5) (layer F.Cu) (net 5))
 (segment (start 135.4963 111.9759) (end 135.4963 114.8334) (width 0.5) (layer F.Cu) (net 5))
 (segment (start 136.2456 115.5827) (end 137.7188 115.5827) (width 0.5) (layer F.Cu) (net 5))
 (segment (start 135.4963 114.8334) (end 136.2456 115.5827) (width 0.5) (layer F.Cu) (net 5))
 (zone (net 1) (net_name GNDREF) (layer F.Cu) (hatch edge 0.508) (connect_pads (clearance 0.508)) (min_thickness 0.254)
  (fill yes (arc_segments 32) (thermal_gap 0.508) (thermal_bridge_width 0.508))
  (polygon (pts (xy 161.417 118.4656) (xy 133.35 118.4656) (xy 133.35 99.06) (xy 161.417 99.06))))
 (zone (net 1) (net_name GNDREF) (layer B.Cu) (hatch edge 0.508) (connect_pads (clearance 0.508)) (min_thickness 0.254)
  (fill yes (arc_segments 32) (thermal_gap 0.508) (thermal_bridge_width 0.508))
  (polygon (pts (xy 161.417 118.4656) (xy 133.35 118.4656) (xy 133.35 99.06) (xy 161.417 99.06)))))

